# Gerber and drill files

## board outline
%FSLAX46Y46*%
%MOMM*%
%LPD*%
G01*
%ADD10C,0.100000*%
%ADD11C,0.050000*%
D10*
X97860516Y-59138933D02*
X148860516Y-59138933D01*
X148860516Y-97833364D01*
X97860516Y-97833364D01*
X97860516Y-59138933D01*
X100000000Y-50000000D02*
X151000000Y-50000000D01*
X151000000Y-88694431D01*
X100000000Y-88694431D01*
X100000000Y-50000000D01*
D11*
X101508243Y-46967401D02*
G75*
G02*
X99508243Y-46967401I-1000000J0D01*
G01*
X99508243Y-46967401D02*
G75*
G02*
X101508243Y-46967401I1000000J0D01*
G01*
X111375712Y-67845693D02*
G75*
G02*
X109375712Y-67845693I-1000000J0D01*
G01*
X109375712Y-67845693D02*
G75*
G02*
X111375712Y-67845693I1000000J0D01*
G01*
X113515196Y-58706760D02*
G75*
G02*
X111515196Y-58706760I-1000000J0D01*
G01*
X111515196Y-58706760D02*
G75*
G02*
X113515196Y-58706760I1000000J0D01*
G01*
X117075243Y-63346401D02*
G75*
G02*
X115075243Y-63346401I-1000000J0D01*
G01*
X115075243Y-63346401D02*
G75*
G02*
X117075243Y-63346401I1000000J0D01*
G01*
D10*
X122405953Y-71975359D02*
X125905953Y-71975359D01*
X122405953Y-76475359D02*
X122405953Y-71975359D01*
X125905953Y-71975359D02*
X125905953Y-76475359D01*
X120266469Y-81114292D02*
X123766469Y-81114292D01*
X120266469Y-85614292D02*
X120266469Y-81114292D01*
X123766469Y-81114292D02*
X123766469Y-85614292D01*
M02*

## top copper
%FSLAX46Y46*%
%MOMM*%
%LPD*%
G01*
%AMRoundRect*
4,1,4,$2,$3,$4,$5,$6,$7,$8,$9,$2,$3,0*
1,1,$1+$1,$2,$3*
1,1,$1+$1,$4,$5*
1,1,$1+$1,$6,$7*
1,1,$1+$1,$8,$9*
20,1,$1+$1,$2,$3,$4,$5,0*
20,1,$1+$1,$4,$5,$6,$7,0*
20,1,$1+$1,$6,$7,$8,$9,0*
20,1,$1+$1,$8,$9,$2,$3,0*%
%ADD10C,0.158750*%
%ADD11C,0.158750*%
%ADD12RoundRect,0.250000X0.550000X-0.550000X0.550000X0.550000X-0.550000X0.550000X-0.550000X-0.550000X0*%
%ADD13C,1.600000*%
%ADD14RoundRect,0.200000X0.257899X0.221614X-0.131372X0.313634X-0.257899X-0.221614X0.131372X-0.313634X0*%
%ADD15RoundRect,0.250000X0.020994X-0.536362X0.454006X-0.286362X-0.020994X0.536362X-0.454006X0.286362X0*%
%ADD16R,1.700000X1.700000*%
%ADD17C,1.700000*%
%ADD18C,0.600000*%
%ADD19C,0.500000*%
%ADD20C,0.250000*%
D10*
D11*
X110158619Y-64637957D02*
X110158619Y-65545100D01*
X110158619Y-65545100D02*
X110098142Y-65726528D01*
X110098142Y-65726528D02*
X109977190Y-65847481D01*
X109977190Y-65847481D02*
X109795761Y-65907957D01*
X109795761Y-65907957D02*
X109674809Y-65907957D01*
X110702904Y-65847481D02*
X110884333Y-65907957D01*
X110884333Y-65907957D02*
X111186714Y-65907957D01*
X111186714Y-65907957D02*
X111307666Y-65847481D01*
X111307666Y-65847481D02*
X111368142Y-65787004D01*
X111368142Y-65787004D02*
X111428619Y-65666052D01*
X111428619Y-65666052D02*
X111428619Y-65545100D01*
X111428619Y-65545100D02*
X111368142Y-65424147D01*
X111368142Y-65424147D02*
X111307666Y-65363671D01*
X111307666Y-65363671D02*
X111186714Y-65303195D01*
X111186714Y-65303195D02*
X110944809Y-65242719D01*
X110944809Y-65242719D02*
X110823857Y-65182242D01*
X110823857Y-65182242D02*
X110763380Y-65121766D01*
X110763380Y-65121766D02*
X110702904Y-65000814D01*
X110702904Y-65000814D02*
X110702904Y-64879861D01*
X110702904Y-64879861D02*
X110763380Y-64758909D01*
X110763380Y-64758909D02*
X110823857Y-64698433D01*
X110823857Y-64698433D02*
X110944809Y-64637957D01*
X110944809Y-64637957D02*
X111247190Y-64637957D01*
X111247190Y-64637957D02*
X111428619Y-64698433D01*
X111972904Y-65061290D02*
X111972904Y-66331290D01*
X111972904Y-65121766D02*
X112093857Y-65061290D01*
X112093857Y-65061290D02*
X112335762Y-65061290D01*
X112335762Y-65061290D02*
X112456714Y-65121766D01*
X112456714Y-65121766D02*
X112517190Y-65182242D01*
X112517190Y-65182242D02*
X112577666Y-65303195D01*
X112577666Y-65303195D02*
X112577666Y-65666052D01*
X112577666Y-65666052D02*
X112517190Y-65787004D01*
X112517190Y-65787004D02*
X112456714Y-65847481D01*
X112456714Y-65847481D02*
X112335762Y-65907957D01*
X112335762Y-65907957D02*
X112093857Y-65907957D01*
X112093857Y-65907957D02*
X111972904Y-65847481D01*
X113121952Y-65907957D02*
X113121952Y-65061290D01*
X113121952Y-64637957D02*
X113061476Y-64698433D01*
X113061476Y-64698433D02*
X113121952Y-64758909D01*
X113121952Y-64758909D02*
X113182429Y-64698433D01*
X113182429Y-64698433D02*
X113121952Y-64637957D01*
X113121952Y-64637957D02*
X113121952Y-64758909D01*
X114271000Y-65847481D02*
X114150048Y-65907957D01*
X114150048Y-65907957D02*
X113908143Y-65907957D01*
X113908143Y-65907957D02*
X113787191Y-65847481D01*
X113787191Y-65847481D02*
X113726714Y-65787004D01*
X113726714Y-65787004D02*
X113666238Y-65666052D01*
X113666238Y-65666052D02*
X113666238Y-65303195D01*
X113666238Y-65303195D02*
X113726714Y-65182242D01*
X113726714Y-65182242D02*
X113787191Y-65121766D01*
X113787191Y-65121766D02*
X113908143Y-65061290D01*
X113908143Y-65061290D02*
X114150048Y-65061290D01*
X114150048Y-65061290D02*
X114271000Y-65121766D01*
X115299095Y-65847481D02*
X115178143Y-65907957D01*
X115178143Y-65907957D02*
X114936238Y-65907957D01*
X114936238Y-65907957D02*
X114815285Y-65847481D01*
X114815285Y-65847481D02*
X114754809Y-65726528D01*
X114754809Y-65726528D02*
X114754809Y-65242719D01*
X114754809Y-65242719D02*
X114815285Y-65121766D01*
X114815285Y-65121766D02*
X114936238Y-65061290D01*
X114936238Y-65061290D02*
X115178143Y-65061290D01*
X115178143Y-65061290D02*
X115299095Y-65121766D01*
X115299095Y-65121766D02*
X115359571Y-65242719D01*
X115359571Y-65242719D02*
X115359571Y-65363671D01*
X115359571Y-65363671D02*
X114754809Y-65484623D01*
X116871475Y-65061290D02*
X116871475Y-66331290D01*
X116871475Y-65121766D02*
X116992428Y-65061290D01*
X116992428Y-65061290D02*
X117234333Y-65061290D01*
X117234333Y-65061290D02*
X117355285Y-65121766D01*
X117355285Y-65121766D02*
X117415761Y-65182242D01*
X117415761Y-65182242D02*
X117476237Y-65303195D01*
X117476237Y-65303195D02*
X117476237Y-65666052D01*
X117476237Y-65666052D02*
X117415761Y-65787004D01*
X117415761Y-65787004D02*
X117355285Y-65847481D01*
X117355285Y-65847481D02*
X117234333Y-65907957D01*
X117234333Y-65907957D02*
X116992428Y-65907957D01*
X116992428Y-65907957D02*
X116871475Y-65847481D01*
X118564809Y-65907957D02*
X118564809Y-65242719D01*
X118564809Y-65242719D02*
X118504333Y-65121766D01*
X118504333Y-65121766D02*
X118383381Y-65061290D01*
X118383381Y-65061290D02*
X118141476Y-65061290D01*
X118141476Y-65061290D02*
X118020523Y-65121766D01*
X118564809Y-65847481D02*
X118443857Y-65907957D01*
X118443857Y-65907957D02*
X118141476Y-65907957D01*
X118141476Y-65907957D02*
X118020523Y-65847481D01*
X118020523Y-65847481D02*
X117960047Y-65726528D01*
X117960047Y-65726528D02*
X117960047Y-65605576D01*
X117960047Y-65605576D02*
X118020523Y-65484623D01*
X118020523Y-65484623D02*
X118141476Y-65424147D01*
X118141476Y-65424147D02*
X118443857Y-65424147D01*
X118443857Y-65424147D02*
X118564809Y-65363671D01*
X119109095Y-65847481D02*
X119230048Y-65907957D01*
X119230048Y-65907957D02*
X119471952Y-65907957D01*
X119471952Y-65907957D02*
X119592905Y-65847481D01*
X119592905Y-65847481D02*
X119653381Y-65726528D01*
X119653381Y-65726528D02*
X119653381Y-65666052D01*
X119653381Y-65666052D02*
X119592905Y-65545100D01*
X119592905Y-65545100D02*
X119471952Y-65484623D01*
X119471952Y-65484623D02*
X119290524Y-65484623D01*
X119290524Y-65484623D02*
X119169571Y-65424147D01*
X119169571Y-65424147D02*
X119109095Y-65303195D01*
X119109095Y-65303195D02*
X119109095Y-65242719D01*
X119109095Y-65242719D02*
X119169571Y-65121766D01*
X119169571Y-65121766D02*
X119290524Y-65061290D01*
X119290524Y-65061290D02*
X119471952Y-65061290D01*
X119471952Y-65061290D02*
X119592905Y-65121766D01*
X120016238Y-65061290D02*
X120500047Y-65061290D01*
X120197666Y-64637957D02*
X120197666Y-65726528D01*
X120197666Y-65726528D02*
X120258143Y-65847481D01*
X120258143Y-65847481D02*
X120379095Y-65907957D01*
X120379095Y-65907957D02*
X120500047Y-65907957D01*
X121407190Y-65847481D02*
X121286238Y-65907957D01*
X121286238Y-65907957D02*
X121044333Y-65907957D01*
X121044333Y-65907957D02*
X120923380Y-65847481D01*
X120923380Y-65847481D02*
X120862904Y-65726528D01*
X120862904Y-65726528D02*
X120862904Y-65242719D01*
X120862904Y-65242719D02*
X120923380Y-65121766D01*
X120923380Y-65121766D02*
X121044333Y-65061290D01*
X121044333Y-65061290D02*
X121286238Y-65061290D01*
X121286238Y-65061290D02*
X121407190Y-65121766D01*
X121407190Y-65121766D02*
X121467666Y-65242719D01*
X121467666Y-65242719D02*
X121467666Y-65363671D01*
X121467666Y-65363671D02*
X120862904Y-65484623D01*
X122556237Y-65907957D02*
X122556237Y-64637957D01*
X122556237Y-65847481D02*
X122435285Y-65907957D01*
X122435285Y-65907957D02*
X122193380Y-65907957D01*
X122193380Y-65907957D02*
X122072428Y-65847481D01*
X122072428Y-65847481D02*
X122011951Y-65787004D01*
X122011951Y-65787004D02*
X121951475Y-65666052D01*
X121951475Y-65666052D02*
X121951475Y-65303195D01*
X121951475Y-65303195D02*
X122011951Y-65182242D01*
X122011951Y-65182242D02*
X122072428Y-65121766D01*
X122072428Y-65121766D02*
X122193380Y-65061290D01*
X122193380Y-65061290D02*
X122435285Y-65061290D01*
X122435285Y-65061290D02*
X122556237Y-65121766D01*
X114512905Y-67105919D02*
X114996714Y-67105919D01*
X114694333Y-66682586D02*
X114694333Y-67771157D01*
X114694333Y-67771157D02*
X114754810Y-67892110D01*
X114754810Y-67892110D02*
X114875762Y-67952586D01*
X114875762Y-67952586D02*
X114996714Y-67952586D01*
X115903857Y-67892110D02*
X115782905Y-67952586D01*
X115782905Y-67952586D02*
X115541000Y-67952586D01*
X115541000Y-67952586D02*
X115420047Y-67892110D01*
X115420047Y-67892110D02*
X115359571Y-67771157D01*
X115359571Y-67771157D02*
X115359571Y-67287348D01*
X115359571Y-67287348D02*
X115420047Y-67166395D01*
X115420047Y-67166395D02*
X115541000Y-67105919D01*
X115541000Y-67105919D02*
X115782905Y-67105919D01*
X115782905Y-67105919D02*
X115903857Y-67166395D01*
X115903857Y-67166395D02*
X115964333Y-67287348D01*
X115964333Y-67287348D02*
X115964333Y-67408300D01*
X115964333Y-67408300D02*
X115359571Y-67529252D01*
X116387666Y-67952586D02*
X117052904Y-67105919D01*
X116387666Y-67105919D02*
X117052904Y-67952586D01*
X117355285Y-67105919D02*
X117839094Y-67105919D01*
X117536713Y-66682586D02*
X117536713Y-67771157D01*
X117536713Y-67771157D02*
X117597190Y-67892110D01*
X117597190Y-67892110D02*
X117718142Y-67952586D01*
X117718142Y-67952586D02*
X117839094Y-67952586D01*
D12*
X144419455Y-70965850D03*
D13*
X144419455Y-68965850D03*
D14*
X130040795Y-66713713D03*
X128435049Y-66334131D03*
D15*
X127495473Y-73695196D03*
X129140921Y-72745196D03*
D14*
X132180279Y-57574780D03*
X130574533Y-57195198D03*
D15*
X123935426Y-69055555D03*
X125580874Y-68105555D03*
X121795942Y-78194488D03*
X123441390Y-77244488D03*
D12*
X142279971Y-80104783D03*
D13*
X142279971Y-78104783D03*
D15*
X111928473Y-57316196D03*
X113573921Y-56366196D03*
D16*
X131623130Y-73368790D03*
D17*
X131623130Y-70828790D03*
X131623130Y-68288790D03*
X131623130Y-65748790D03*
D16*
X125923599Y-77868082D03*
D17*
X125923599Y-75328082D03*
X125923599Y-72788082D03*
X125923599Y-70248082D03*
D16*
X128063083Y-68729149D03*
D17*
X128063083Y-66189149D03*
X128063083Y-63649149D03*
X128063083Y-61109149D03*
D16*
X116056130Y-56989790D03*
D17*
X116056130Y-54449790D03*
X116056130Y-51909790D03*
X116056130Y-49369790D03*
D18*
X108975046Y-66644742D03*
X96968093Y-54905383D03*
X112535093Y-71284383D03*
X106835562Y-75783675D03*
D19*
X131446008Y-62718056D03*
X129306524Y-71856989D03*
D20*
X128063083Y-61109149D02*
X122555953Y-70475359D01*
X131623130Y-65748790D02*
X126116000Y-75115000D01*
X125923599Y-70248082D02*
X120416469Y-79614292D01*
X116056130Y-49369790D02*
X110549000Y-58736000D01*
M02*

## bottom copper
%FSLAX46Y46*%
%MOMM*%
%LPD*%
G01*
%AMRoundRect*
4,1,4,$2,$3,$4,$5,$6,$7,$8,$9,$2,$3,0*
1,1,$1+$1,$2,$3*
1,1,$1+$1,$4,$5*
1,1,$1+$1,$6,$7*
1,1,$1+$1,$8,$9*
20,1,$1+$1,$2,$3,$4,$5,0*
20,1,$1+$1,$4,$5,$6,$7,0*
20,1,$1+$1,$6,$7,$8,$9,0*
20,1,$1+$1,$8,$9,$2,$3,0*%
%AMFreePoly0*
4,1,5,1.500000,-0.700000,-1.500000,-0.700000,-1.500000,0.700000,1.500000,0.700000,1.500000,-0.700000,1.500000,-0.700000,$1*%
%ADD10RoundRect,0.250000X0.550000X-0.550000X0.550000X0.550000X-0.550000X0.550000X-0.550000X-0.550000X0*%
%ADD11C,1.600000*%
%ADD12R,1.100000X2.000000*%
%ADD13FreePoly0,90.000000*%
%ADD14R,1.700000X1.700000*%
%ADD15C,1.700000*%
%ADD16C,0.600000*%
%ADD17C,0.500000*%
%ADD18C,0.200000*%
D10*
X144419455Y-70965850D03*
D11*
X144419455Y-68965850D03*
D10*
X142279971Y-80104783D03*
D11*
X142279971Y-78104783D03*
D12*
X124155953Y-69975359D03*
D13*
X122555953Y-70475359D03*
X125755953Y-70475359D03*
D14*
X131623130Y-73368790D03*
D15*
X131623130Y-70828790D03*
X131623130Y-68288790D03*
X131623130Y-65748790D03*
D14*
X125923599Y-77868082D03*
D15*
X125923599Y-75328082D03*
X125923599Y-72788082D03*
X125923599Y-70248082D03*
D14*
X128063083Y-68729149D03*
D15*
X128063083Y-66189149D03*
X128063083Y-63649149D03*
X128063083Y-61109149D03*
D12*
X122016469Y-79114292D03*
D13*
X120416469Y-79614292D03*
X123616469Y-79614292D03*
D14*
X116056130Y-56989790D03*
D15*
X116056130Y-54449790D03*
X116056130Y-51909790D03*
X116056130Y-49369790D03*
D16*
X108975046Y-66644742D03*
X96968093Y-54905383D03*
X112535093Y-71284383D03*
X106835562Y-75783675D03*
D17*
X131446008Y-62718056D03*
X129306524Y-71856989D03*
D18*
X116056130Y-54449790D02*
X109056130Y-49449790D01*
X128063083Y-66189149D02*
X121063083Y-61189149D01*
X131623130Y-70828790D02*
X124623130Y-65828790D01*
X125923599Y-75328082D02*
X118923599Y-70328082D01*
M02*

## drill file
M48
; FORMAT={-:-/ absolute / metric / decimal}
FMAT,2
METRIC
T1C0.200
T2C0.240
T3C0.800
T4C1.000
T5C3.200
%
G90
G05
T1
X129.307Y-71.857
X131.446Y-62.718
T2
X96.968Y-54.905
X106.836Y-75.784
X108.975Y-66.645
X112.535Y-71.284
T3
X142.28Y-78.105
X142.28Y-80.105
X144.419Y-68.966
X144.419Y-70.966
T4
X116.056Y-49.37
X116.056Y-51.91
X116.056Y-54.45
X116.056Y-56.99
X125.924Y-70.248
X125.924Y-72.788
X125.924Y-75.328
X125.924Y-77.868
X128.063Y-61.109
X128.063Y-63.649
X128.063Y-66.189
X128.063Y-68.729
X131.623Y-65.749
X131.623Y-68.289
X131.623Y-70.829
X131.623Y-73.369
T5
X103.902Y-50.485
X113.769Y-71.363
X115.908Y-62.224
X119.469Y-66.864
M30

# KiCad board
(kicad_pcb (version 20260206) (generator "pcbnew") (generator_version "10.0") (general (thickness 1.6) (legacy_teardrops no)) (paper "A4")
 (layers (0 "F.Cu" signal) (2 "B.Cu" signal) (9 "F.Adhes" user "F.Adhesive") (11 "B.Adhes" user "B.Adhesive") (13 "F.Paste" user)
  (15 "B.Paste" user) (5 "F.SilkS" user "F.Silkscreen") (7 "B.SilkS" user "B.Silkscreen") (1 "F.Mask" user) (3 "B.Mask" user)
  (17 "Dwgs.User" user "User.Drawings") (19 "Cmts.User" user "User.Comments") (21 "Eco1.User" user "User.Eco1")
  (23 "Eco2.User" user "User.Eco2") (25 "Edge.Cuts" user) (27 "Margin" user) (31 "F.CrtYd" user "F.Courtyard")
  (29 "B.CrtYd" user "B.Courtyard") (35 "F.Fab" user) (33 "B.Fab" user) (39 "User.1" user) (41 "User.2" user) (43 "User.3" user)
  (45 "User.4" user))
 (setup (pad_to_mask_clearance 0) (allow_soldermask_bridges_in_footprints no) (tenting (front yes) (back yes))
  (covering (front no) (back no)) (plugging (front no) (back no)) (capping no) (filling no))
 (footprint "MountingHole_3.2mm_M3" (layer "F.Cu") (at 103.901531 50.484708 45)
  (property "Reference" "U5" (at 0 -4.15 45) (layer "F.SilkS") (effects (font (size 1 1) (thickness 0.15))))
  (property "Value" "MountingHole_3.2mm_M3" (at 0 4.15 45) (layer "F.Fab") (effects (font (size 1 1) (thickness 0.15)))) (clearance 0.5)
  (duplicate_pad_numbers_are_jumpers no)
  (pad "" np_thru_hole circle (at 0 0 45) (size 3.2 3.2) (drill 3.2) (layers "*.Cu" "*.Mask")))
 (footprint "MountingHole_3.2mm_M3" (layer "F.Cu") (at 119.468531 66.863708 45)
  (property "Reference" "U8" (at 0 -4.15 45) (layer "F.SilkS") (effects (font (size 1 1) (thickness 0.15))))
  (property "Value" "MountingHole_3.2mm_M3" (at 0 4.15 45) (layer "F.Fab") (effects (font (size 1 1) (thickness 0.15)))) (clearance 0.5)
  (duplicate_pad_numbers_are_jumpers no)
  (pad "" np_thru_hole circle (at 0 0 45) (size 3.2 3.2) (drill 3.2) (layers "*.Cu" "*.Mask")))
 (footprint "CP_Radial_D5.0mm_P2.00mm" (layer "F.Cu") (at 144.419455 70.96585 90)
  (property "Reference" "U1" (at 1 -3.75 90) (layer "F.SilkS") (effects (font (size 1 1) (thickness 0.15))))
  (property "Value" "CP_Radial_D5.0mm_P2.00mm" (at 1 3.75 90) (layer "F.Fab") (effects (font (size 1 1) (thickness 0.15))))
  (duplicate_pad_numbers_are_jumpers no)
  (pad "1" thru_hole roundrect (at 0 0 90) (size 1.6 1.6) (drill 0.8) (layers "*.Cu" "*.Mask") (remove_unused_layers no)
   (roundrect_rratio 0.15625) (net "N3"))
  (pad "2" thru_hole circle (at 2 0 90) (size 1.6 1.6) (drill 0.8) (layers "*.Cu" "*.Mask") (remove_unused_layers no) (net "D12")))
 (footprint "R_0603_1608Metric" (layer "F.Cu") (at 129.237922 66.523922 166.7)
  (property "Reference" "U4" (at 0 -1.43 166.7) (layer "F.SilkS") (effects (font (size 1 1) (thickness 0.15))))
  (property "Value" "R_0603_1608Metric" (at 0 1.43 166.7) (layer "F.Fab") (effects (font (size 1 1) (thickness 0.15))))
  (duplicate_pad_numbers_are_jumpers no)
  (pad "1" smd roundrect (at -0.825 0 166.7) (size 0.8 0.95) (layers "F.Cu" "F.Mask" "F.Paste") (roundrect_rratio 0.25) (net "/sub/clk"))
  (pad "2" smd roundrect (at 0.825 0 166.7) (size 0.8 0.95) (layers "F.Cu" "F.Mask" "F.Paste") (roundrect_rratio 0.25) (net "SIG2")))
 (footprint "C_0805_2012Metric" (layer "F.Cu") (at 128.318197 73.220196 30)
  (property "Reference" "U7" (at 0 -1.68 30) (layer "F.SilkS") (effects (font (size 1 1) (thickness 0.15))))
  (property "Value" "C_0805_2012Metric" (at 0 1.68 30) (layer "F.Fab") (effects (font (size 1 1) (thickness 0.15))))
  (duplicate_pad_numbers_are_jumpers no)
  (pad "1" smd roundrect (at -0.95 0 30) (size 1 1.45) (layers "F.Cu" "F.Mask" "F.Paste") (roundrect_rratio 0.25) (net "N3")
   (clearance 0.35))
  (pad "2" smd roundrect (at 0.95 0 30) (size 1 1.45) (layers "F.Cu" "F.Mask" "F.Paste") (roundrect_rratio 0.25)))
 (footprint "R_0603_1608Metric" (layer "F.Cu") (at 131.377406 57.384989 166.7)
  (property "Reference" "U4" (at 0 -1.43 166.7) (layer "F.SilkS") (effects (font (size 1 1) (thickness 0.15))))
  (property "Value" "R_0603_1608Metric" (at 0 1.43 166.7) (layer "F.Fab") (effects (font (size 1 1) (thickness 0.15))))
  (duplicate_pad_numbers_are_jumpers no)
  (pad "1" smd roundrect (at -0.825 0 166.7) (size 0.8 0.95) (layers "F.Cu" "F.Mask" "F.Paste") (roundrect_rratio 0.25) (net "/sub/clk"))
  (pad "2" smd roundrect (at 0.825 0 166.7) (size 0.8 0.95) (layers "F.Cu" "F.Mask" "F.Paste") (roundrect_rratio 0.25) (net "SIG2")))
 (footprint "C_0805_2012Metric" (layer "F.Cu") (at 124.75815 68.580555 30)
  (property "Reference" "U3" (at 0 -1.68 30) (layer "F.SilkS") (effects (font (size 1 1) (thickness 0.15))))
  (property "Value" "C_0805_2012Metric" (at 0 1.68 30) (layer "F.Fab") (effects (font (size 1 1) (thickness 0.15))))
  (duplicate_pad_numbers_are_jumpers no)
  (pad "1" smd roundrect (at -0.95 0 30) (size 1 1.45) (layers "F.Cu" "F.Mask" "F.Paste") (roundrect_rratio 0.25) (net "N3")
   (clearance 0.35))
  (pad "2" smd roundrect (at 0.95 0 30) (size 1 1.45) (layers "F.Cu" "F.Mask" "F.Paste") (roundrect_rratio 0.25)))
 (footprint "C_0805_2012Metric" (layer "F.Cu") (at 122.618666 77.719488 30)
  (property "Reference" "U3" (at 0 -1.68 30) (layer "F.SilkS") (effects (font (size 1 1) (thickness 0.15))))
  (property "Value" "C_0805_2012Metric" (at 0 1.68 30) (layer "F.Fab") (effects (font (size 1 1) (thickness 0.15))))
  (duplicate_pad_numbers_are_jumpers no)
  (pad "1" smd roundrect (at -0.95 0 30) (size 1 1.45) (layers "F.Cu" "F.Mask" "F.Paste") (roundrect_rratio 0.25) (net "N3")
   (clearance 0.35))
  (pad "2" smd roundrect (at 0.95 0 30) (size 1 1.45) (layers "F.Cu" "F.Mask" "F.Paste") (roundrect_rratio 0.25)))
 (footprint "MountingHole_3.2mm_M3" (layer "F.Cu") (at 113.769 71.363 45)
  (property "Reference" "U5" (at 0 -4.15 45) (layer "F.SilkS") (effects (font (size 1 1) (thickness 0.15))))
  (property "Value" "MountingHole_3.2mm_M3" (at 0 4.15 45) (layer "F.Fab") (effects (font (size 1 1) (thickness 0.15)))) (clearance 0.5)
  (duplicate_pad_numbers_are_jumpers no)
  (pad "" np_thru_hole circle (at 0 0 45) (size 3.2 3.2) (drill 3.2) (layers "*.Cu" "*.Mask")))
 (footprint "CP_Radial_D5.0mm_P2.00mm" (layer "F.Cu") (at 142.279971 80.104783 90)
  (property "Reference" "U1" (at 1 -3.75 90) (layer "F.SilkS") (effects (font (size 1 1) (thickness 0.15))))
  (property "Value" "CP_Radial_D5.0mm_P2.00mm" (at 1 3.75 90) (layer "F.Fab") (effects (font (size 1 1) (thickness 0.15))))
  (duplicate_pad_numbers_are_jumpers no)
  (pad "1" thru_hole roundrect (at 0 0 90) (size 1.6 1.6) (drill 0.8) (layers "*.Cu" "*.Mask") (remove_unused_layers no)
   (roundrect_rratio 0.15625) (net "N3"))
  (pad "2" thru_hole circle (at 2 0 90) (size 1.6 1.6) (drill 0.8) (layers "*.Cu" "*.Mask") (remove_unused_layers no) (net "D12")))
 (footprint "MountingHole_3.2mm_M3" (layer "F.Cu") (at 115.908484 62.224067 45)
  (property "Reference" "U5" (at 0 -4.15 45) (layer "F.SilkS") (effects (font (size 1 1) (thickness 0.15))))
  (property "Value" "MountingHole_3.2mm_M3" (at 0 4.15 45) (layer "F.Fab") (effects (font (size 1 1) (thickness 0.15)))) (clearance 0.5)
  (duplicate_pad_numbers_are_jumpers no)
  (pad "" np_thru_hole circle (at 0 0 45) (size 3.2 3.2) (drill 3.2) (layers "*.Cu" "*.Mask")))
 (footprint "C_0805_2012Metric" (layer "F.Cu") (at 112.751197 56.841196 30)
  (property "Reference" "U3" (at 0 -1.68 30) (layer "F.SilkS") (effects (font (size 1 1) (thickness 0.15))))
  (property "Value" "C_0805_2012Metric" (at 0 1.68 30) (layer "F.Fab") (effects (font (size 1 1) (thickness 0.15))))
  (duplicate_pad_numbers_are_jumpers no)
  (pad "1" smd roundrect (at -0.95 0 30) (size 1 1.45) (layers "F.Cu" "F.Mask" "F.Paste") (roundrect_rratio 0.25) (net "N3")
   (clearance 0.35))
  (pad "2" smd roundrect (at 0.95 0 30) (size 1 1.45) (layers "F.Cu" "F.Mask" "F.Paste") (roundrect_rratio 0.25)))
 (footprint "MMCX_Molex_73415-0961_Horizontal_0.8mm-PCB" (layer "B.Cu") (at 124.155953 72.725359 90)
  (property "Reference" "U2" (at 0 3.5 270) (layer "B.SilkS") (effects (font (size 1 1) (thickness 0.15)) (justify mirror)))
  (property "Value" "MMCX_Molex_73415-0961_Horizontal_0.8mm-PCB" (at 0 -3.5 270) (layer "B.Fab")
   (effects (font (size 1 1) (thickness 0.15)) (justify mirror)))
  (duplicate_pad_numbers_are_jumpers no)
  (fp_line (start 0.75 -1.75) (end 0.75 1.75) (stroke (width 0.1) (type solid)) (layer "Edge.Cuts"))
  (fp_line (start -3.75 -1.75) (end 0.75 -1.75) (stroke (width 0.1) (type solid)) (layer "Edge.Cuts"))
  (fp_line (start 0.75 1.75) (end -3.75 1.75) (stroke (width 0.1) (type solid)) (layer "Edge.Cuts"))
  (pad "1" smd rect (at 2.75 0 90) (size 2 1.1) (layers "B.Cu" "B.Mask" "B.Paste") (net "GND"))
  (pad "2" smd custom (at 2.25 -1.6 90) (size 3 1.4) (layers "B.Cu" "B.Mask" "B.Paste") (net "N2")
   (options (clearance outline) (anchor rect)) (primitives))
  (pad "2" smd custom (at 2.25 1.6 90) (size 3 1.4) (layers "B.Cu" "B.Mask" "B.Paste") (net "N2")
   (options (clearance outline) (anchor rect)) (primitives)))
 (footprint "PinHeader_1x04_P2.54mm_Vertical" (layer "B.Cu") (at 131.62313 73.36879)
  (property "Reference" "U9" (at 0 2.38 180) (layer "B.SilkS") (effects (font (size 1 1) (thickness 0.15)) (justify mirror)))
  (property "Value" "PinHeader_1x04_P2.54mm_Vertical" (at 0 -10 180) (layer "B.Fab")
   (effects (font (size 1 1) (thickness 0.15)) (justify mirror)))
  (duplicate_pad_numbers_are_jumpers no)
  (pad "1" thru_hole rect (at 0 0) (size 1.7 1.7) (drill 1) (layers "*.Cu" "*.Mask") (remove_unused_layers no) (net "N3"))
  (pad "2" thru_hole circle (at 0 -2.54) (size 1.7 1.7) (drill 1) (layers "*.Cu" "*.Mask") (remove_unused_layers no) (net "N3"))
  (pad "3" thru_hole circle (at 0 -5.08) (size 1.7 1.7) (drill 1) (layers "*.Cu" "*.Mask") (remove_unused_layers no) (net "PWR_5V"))
  (pad "4" thru_hole circle (at 0 -7.62) (size 1.7 1.7) (drill 1) (layers "*.Cu" "*.Mask") (remove_unused_layers no)))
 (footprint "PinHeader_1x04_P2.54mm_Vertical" (layer "B.Cu") (at 125.923599 77.868082)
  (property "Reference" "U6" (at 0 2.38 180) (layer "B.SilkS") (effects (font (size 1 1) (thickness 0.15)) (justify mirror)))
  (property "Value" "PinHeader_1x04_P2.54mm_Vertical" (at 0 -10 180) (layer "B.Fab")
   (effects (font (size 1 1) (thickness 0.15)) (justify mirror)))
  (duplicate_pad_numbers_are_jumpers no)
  (pad "1" thru_hole rect (at 0 0) (size 1.7 1.7) (drill 1) (layers "*.Cu" "*.Mask") (remove_unused_layers no) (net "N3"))
  (pad "2" thru_hole circle (at 0 -2.54) (size 1.7 1.7) (drill 1) (layers "*.Cu" "*.Mask") (remove_unused_layers no) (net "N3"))
  (pad "3" thru_hole circle (at 0 -5.08) (size 1.7 1.7) (drill 1) (layers "*.Cu" "*.Mask") (remove_unused_layers no) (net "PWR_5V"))
  (pad "4" thru_hole circle (at 0 -7.62) (size 1.7 1.7) (drill 1) (layers "*.Cu" "*.Mask") (remove_unused_layers no)))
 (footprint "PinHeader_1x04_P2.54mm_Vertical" (layer "B.Cu") (at 128.063083 68.729149)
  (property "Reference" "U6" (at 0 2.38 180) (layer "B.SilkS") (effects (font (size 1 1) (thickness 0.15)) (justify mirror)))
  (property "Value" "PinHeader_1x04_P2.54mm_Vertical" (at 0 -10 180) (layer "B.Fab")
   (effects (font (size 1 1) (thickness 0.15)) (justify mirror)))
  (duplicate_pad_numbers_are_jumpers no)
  (pad "1" thru_hole rect (at 0 0) (size 1.7 1.7) (drill 1) (layers "*.Cu" "*.Mask") (remove_unused_layers no) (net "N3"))
  (pad "2" thru_hole circle (at 0 -2.54) (size 1.7 1.7) (drill 1) (layers "*.Cu" "*.Mask") (remove_unused_layers no) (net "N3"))
  (pad "3" thru_hole circle (at 0 -5.08) (size 1.7 1.7) (drill 1) (layers "*.Cu" "*.Mask") (remove_unused_layers no) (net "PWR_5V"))
  (pad "4" thru_hole circle (at 0 -7.62) (size 1.7 1.7) (drill 1) (layers "*.Cu" "*.Mask") (remove_unused_layers no)))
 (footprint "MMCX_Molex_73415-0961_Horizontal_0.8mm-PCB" (layer "B.Cu") (at 122.016469 81.864292 90)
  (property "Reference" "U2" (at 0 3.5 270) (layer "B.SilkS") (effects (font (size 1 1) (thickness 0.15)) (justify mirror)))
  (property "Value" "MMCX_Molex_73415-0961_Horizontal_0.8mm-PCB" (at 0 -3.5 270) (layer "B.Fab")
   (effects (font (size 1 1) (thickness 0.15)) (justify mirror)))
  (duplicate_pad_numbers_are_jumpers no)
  (fp_line (start 0.75 -1.75) (end 0.75 1.75) (stroke (width 0.1) (type solid)) (layer "Edge.Cuts"))
  (fp_line (start -3.75 -1.75) (end 0.75 -1.75) (stroke (width 0.1) (type solid)) (layer "Edge.Cuts"))
  (fp_line (start 0.75 1.75) (end -3.75 1.75) (stroke (width 0.1) (type solid)) (layer "Edge.Cuts"))
  (pad "1" smd rect (at 2.75 0 90) (size 2 1.1) (layers "B.Cu" "B.Mask" "B.Paste") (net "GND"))
  (pad "2" smd custom (at 2.25 -1.6 90) (size 3 1.4) (layers "B.Cu" "B.Mask" "B.Paste") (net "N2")
   (options (clearance outline) (anchor rect)) (primitives))
  (pad "2" smd custom (at 2.25 1.6 90) (size 3 1.4) (layers "B.Cu" "B.Mask" "B.Paste") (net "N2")
   (options (clearance outline) (anchor rect)) (primitives)))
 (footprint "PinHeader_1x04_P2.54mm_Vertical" (layer "B.Cu") (at 116.05613 56.98979)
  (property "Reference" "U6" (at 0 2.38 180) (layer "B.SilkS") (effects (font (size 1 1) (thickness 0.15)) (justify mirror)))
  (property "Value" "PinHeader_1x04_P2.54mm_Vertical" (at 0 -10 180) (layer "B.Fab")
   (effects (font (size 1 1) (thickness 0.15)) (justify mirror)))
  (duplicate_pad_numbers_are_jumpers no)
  (pad "1" thru_hole rect (at 0 0) (size 1.7 1.7) (drill 1) (layers "*.Cu" "*.Mask") (remove_unused_layers no) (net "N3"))
  (pad "2" thru_hole circle (at 0 -2.54) (size 1.7 1.7) (drill 1) (layers "*.Cu" "*.Mask") (remove_unused_layers no) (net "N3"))
  (pad "3" thru_hole circle (at 0 -5.08) (size 1.7 1.7) (drill 1) (layers "*.Cu" "*.Mask") (remove_unused_layers no) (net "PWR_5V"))
  (pad "4" thru_hole circle (at 0 -7.62) (size 1.7 1.7) (drill 1) (layers "*.Cu" "*.Mask") (remove_unused_layers no)))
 (gr_rect (start 97.860516 59.138933) (end 148.860516 97.833364) (stroke (width 0.1) (type default)) (fill no) (layer "Edge.Cuts"))
 (gr_rect (start 100 50) (end 151 88.694431) (stroke (width 0.1) (type default)) (fill no) (layer "Edge.Cuts"))
 (gr_circle (center 100.508243 46.967401) (end 101.508243 46.967401) (stroke (width 0.05) (type default)) (fill no) (layer "Edge.Cuts"))
 (gr_circle (center 110.375712 67.845693) (end 111.375712 67.845693) (stroke (width 0.05) (type default)) (fill no) (layer "Edge.Cuts"))
 (gr_circle (center 112.515196 58.70676) (end 113.515196 58.70676) (stroke (width 0.05) (type default)) (fill no) (layer "Edge.Cuts"))
 (gr_circle (center 116.075243 63.346401) (end 117.075243 63.346401) (stroke (width 0.05) (type default)) (fill no) (layer "Edge.Cuts"))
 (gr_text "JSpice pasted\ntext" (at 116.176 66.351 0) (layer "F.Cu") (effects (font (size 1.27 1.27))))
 (segment (start 128.063083 61.109149) (end 122.555953 70.475359) (width 0.25) (layer "F.Cu") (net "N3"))
 (segment (start 131.62313 65.74879) (end 126.116 75.115) (width 0.25) (layer "F.Cu") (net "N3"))
 (segment (start 125.923599 70.248082) (end 120.416469 79.614292) (width 0.25) (layer "F.Cu") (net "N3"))
 (segment (start 116.05613 49.36979) (end 110.549 58.736) (width 0.25) (layer "F.Cu") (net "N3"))
 (segment (start 116.05613 54.44979) (end 109.05613 49.44979) (width 0.2) (layer "B.Cu") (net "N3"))
 (segment (start 128.063083 66.189149) (end 121.063083 61.189149) (width 0.2) (layer "B.Cu") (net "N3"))
 (segment (start 131.62313 70.82879) (end 124.62313 65.82879) (width 0.2) (layer "B.Cu") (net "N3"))
 (segment (start 125.923599 75.328082) (end 118.923599 70.328082) (width 0.2) (layer "B.Cu") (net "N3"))
 (via (at 108.975046 66.644742) (size 0.6) (drill 0.24) (layers "F.Cu" "B.Cu") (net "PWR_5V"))
 (via (at 96.968093 54.905383) (size 0.6) (drill 0.24) (layers "F.Cu" "B.Cu") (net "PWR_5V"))
 (via (at 112.535093 71.284383) (size 0.6) (drill 0.24) (layers "F.Cu" "B.Cu") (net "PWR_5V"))
 (via (at 106.835562 75.783675) (size 0.6) (drill 0.24) (layers "F.Cu" "B.Cu") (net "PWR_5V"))
 (via (at 131.446008 62.718056) (size 0.5) (drill 0.2) (layers "F.Cu" "B.Cu") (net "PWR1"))
 (via (at 129.306524 71.856989) (size 0.5) (drill 0.2) (layers "F.Cu" "B.Cu") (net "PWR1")))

